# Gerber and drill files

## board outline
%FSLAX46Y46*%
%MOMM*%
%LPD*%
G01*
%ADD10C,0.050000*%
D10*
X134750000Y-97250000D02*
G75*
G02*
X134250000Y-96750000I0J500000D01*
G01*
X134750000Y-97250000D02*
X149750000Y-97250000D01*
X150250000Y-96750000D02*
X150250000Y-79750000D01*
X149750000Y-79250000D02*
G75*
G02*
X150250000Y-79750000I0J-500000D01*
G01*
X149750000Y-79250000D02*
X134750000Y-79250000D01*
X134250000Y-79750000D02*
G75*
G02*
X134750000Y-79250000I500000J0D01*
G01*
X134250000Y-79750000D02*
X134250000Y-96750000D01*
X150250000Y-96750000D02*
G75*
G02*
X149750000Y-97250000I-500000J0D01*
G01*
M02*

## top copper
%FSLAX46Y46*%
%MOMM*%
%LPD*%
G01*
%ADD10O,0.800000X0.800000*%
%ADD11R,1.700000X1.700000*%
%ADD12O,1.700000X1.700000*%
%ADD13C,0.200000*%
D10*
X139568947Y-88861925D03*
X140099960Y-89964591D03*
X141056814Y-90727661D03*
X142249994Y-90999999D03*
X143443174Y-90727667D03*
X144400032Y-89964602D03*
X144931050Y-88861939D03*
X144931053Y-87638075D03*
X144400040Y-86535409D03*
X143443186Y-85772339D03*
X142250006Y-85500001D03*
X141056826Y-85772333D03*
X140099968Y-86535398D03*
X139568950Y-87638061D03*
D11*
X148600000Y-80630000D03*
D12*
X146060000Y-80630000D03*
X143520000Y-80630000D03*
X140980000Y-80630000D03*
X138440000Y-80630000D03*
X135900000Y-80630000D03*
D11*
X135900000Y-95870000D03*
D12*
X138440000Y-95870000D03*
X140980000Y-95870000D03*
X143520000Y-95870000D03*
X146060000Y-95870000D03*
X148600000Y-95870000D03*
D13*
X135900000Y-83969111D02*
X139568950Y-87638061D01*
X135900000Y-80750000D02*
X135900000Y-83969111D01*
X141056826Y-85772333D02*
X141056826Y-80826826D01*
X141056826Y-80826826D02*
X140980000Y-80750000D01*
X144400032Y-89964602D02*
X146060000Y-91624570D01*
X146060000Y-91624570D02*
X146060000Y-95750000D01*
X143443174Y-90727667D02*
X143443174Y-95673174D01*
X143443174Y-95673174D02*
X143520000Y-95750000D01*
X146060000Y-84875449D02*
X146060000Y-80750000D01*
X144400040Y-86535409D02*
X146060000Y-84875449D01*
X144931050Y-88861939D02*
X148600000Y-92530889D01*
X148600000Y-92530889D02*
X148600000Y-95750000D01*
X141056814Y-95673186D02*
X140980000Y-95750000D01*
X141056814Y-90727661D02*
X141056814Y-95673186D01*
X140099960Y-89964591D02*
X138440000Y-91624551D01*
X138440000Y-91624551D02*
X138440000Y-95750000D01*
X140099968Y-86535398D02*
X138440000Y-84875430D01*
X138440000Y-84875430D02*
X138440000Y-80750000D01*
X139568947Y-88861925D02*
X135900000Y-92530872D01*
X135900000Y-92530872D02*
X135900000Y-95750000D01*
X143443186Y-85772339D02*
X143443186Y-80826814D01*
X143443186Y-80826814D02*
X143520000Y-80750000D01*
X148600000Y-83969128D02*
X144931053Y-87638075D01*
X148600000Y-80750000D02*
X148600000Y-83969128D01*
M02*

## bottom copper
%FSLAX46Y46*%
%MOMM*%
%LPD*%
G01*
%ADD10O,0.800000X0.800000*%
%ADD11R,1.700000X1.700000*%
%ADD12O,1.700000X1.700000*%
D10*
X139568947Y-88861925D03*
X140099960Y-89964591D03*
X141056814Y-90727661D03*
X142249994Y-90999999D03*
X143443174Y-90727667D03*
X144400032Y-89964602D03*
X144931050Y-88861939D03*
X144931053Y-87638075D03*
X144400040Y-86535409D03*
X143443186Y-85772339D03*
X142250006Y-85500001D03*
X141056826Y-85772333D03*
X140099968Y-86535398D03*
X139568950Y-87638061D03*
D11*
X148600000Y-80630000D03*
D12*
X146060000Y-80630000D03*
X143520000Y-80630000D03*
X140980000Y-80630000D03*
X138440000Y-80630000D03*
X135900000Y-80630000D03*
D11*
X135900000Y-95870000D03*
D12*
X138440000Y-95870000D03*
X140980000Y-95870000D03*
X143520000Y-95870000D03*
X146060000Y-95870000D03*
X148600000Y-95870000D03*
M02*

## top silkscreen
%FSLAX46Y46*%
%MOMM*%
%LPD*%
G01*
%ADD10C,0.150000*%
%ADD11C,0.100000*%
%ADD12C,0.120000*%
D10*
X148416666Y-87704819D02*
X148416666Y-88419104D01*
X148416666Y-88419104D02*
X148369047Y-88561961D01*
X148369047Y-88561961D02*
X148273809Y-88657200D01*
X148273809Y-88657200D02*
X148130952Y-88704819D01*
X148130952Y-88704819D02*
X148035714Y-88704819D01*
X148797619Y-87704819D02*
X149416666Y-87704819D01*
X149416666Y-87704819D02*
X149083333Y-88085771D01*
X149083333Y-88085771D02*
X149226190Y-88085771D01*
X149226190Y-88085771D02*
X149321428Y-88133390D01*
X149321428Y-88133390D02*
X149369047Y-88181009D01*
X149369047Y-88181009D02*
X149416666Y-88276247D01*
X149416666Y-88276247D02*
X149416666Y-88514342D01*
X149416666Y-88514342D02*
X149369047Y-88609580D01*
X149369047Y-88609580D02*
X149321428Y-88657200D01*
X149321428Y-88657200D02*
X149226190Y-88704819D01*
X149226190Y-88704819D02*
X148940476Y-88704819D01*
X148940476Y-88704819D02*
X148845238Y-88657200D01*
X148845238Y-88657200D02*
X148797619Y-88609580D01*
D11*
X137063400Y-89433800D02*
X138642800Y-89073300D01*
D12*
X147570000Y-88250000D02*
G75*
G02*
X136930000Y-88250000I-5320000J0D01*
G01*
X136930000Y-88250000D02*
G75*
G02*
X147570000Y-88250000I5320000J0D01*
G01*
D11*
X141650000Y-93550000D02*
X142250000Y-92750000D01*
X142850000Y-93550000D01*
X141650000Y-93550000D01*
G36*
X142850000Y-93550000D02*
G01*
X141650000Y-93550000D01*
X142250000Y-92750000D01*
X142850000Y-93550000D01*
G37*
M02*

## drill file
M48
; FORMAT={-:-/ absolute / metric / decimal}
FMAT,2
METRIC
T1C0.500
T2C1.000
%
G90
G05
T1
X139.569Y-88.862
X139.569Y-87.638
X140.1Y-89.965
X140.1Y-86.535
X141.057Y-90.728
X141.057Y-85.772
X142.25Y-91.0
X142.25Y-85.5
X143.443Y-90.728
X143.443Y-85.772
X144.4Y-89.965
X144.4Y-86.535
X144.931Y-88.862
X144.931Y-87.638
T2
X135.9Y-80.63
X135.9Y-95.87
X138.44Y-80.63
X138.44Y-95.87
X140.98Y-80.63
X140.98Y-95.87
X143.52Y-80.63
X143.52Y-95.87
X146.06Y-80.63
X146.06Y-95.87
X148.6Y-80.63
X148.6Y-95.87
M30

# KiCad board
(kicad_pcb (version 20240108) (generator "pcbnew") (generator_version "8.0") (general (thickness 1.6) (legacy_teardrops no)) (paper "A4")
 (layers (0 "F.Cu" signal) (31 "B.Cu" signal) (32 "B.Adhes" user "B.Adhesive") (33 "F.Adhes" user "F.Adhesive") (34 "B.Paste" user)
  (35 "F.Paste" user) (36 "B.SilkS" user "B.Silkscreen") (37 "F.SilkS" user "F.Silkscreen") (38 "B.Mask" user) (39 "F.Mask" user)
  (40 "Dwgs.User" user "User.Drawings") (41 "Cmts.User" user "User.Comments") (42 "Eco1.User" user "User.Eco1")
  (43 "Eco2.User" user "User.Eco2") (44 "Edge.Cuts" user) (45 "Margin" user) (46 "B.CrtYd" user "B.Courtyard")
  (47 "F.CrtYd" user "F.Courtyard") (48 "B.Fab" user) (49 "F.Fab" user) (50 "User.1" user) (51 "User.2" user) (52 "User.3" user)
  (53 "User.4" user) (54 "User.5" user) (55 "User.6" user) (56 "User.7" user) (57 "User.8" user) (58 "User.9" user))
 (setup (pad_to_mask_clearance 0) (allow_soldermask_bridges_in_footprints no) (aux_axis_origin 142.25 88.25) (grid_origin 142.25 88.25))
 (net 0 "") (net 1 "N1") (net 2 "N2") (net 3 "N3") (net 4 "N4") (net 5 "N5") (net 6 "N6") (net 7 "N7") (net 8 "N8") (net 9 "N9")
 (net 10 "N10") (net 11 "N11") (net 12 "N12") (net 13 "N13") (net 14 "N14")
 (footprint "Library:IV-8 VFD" (layer "F.Cu") (at 142.25 88.25)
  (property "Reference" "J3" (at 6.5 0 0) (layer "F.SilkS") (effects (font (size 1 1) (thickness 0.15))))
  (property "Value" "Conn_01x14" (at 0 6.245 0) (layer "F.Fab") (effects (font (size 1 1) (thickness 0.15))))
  (fp_line (start -5.1866 1.1838) (end -3.6072 0.8233) (stroke (width 0.1) (type default)) (layer "F.SilkS"))
  (fp_circle (center 0 0) (end 0 5.32) (stroke (width 0.12) (type default)) (fill none) (layer "F.SilkS"))
  (fp_poly (pts (xy -0.6 5.3) (xy 0 4.5) (xy 0.6 5.3)) (stroke (width 0.1) (type solid)) (fill solid) (layer "F.SilkS"))
  (pad "1" thru_hole oval (at -2.681053 0.611925) (size 0.8 0.8) (drill 0.5) (layers "*.Cu" "*.Mask") (remove_unused_layers no) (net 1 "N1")
   (thermal_bridge_angle 45))
  (pad "2" thru_hole oval (at -2.15004 1.714591) (size 0.8 0.8) (drill 0.5) (layers "*.Cu" "*.Mask") (remove_unused_layers no) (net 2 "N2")
   (thermal_bridge_angle 45))
  (pad "3" thru_hole oval (at -1.193186 2.477661) (size 0.8 0.8) (drill 0.5) (layers "*.Cu" "*.Mask") (remove_unused_layers no) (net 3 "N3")
   (thermal_bridge_angle 45))
  (pad "4" thru_hole oval (at -0.000006 2.749999) (size 0.8 0.8) (drill 0.5) (layers "*.Cu" "*.Mask") (remove_unused_layers no) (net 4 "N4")
   (thermal_bridge_angle 45))
  (pad "5" thru_hole oval (at 1.193174 2.477667) (size 0.8 0.8) (drill 0.5) (layers "*.Cu" "*.Mask") (remove_unused_layers no) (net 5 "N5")
   (thermal_bridge_angle 45))
  (pad "6" thru_hole oval (at 2.150032 1.714602) (size 0.8 0.8) (drill 0.5) (layers "*.Cu" "*.Mask") (remove_unused_layers no) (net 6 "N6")
   (thermal_bridge_angle 45))
  (pad "7" thru_hole oval (at 2.68105 0.611939) (size 0.8 0.8) (drill 0.5) (layers "*.Cu" "*.Mask") (remove_unused_layers no) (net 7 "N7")
   (thermal_bridge_angle 45))
  (pad "8" thru_hole oval (at 2.681053 -0.611925) (size 0.8 0.8) (drill 0.5) (layers "*.Cu" "*.Mask") (remove_unused_layers no) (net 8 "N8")
   (thermal_bridge_angle 45))
  (pad "9" thru_hole oval (at 2.15004 -1.714591) (size 0.8 0.8) (drill 0.5) (layers "*.Cu" "*.Mask") (remove_unused_layers no) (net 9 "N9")
   (thermal_bridge_angle 45))
  (pad "10" thru_hole oval (at 1.193186 -2.477661) (size 0.8 0.8) (drill 0.5) (layers "*.Cu" "*.Mask") (remove_unused_layers no)
   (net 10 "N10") (thermal_bridge_angle 45))
  (pad "11" thru_hole oval (at 0.000006 -2.749999) (size 0.8 0.8) (drill 0.5) (layers "*.Cu" "*.Mask") (remove_unused_layers no)
   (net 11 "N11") (thermal_bridge_angle 45))
  (pad "12" thru_hole oval (at -1.193174 -2.477667) (size 0.8 0.8) (drill 0.5) (layers "*.Cu" "*.Mask") (remove_unused_layers no)
   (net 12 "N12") (thermal_bridge_angle 45))
  (pad "13" thru_hole oval (at -2.150032 -1.714602) (size 0.8 0.8) (drill 0.5) (layers "*.Cu" "*.Mask") (remove_unused_layers no)
   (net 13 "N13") (thermal_bridge_angle 45))
  (pad "14" thru_hole oval (at -2.68105 -0.611939) (size 0.8 0.8) (drill 0.5) (layers "*.Cu" "*.Mask") (remove_unused_layers no)
   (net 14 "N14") (thermal_bridge_angle 45)))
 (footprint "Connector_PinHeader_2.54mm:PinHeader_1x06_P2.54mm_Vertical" (layer "B.Cu") (at 148.6 80.63 90)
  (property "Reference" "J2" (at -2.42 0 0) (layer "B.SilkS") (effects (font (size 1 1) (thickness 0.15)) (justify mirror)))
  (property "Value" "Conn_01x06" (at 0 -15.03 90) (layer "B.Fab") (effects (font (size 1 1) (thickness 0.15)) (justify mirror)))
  (pad "1" thru_hole rect (at 0 0 90) (size 1.7 1.7) (drill 1) (layers "*.Cu" "*.Mask") (remove_unused_layers no) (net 8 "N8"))
  (pad "2" thru_hole oval (at 0 -2.54 90) (size 1.7 1.7) (drill 1) (layers "*.Cu" "*.Mask") (remove_unused_layers no) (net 9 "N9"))
  (pad "3" thru_hole oval (at 0 -5.08 90) (size 1.7 1.7) (drill 1) (layers "*.Cu" "*.Mask") (remove_unused_layers no) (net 10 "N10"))
  (pad "4" thru_hole oval (at 0 -7.62 90) (size 1.7 1.7) (drill 1) (layers "*.Cu" "*.Mask") (remove_unused_layers no) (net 12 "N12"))
  (pad "5" thru_hole oval (at 0 -10.16 90) (size 1.7 1.7) (drill 1) (layers "*.Cu" "*.Mask") (remove_unused_layers no) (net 13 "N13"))
  (pad "6" thru_hole oval (at 0 -12.7 90) (size 1.7 1.7) (drill 1) (layers "*.Cu" "*.Mask") (remove_unused_layers no) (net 14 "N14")))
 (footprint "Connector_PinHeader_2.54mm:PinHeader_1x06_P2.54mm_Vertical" (layer "B.Cu") (at 135.9 95.87 -90)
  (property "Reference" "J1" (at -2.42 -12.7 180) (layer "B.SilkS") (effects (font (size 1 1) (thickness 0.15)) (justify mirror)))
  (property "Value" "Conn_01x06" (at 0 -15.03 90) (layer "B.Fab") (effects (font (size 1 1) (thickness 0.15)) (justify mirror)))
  (pad "1" thru_hole rect (at 0 0 270) (size 1.7 1.7) (drill 1) (layers "*.Cu" "*.Mask") (remove_unused_layers no) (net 1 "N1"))
  (pad "2" thru_hole oval (at 0 -2.54 270) (size 1.7 1.7) (drill 1) (layers "*.Cu" "*.Mask") (remove_unused_layers no) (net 2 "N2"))
  (pad "3" thru_hole oval (at 0 -5.08 270) (size 1.7 1.7) (drill 1) (layers "*.Cu" "*.Mask") (remove_unused_layers no) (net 3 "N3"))
  (pad "4" thru_hole oval (at 0 -7.62 270) (size 1.7 1.7) (drill 1) (layers "*.Cu" "*.Mask") (remove_unused_layers no) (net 5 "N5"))
  (pad "5" thru_hole oval (at 0 -10.16 270) (size 1.7 1.7) (drill 1) (layers "*.Cu" "*.Mask") (remove_unused_layers no) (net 6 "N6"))
  (pad "6" thru_hole oval (at 0 -12.7 270) (size 1.7 1.7) (drill 1) (layers "*.Cu" "*.Mask") (remove_unused_layers no) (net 7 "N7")))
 (gr_arc (start 134.75 97.25) (mid 134.396447 97.103553) (end 134.25 96.75) (stroke (width 0.05) (type default)) (layer "Edge.Cuts"))
 (gr_line (start 134.75 97.25) (end 149.75 97.25) (stroke (width 0.05) (type default)) (layer "Edge.Cuts"))
 (gr_line (start 150.25 96.75) (end 150.25 79.75) (stroke (width 0.05) (type default)) (layer "Edge.Cuts"))
 (gr_arc (start 149.75 79.25) (mid 150.103553 79.396447) (end 150.25 79.75) (stroke (width 0.05) (type default)) (layer "Edge.Cuts"))
 (gr_line (start 149.75 79.25) (end 134.75 79.25) (stroke (width 0.05) (type default)) (layer "Edge.Cuts"))
 (gr_arc (start 134.25 79.75) (mid 134.396447 79.396447) (end 134.75 79.25) (stroke (width 0.05) (type default)) (layer "Edge.Cuts"))
 (gr_line (start 134.25 79.75) (end 134.25 96.75) (stroke (width 0.05) (type default)) (layer "Edge.Cuts"))
 (gr_arc (start 150.25 96.75) (mid 150.103553 97.103553) (end 149.75 97.25) (stroke (width 0.05) (type default)) (layer "Edge.Cuts"))
 (segment (start 135.9 83.969111) (end 139.56895 87.638061) (width 0.2) (layer "F.Cu") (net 14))
 (segment (start 135.9 80.75) (end 135.9 83.969111) (width 0.2) (layer "F.Cu") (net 14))
 (segment (start 141.056826 85.772333) (end 141.056826 80.826826) (width 0.2) (layer "F.Cu") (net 12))
 (segment (start 141.056826 80.826826) (end 140.98 80.75) (width 0.2) (layer "F.Cu") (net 12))
 (segment (start 144.400032 89.964602) (end 146.06 91.62457) (width 0.2) (layer "F.Cu") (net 6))
 (segment (start 146.06 91.62457) (end 146.06 95.75) (width 0.2) (layer "F.Cu") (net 6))
 (segment (start 143.443174 90.727667) (end 143.443174 95.673174) (width 0.2) (layer "F.Cu") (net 5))
 (segment (start 143.443174 95.673174) (end 143.52 95.75) (width 0.2) (layer "F.Cu") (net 5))
 (segment (start 146.06 84.875449) (end 146.06 80.75) (width 0.2) (layer "F.Cu") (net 9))
 (segment (start 144.40004 86.535409) (end 146.06 84.875449) (width 0.2) (layer "F.Cu") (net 9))
 (segment (start 144.93105 88.861939) (end 148.6 92.530889) (width 0.2) (layer "F.Cu") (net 7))
 (segment (start 148.6 92.530889) (end 148.6 95.75) (width 0.2) (layer "F.Cu") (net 7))
 (segment (start 141.056814 95.673186) (end 140.98 95.75) (width 0.2) (layer "F.Cu") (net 3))
 (segment (start 141.056814 90.727661) (end 141.056814 95.673186) (width 0.2) (layer "F.Cu") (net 3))
 (segment (start 140.09996 89.964591) (end 138.44 91.624551) (width 0.2) (layer "F.Cu") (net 2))
 (segment (start 138.44 91.624551) (end 138.44 95.75) (width 0.2) (layer "F.Cu") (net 2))
 (segment (start 140.099968 86.535398) (end 138.44 84.87543) (width 0.2) (layer "F.Cu") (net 13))
 (segment (start 138.44 84.87543) (end 138.44 80.75) (width 0.2) (layer "F.Cu") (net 13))
 (segment (start 139.568947 88.861925) (end 135.9 92.530872) (width 0.2) (layer "F.Cu") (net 1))
 (segment (start 135.9 92.530872) (end 135.9 95.75) (width 0.2) (layer "F.Cu") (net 1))
 (segment (start 143.443186 85.772339) (end 143.443186 80.826814) (width 0.2) (layer "F.Cu") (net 10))
 (segment (start 143.443186 80.826814) (end 143.52 80.75) (width 0.2) (layer "F.Cu") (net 10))
 (segment (start 148.6 83.969128) (end 144.931053 87.638075) (width 0.2) (layer "F.Cu") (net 8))
 (segment (start 148.6 80.75) (end 148.6 83.969128) (width 0.2) (layer "F.Cu") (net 8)))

